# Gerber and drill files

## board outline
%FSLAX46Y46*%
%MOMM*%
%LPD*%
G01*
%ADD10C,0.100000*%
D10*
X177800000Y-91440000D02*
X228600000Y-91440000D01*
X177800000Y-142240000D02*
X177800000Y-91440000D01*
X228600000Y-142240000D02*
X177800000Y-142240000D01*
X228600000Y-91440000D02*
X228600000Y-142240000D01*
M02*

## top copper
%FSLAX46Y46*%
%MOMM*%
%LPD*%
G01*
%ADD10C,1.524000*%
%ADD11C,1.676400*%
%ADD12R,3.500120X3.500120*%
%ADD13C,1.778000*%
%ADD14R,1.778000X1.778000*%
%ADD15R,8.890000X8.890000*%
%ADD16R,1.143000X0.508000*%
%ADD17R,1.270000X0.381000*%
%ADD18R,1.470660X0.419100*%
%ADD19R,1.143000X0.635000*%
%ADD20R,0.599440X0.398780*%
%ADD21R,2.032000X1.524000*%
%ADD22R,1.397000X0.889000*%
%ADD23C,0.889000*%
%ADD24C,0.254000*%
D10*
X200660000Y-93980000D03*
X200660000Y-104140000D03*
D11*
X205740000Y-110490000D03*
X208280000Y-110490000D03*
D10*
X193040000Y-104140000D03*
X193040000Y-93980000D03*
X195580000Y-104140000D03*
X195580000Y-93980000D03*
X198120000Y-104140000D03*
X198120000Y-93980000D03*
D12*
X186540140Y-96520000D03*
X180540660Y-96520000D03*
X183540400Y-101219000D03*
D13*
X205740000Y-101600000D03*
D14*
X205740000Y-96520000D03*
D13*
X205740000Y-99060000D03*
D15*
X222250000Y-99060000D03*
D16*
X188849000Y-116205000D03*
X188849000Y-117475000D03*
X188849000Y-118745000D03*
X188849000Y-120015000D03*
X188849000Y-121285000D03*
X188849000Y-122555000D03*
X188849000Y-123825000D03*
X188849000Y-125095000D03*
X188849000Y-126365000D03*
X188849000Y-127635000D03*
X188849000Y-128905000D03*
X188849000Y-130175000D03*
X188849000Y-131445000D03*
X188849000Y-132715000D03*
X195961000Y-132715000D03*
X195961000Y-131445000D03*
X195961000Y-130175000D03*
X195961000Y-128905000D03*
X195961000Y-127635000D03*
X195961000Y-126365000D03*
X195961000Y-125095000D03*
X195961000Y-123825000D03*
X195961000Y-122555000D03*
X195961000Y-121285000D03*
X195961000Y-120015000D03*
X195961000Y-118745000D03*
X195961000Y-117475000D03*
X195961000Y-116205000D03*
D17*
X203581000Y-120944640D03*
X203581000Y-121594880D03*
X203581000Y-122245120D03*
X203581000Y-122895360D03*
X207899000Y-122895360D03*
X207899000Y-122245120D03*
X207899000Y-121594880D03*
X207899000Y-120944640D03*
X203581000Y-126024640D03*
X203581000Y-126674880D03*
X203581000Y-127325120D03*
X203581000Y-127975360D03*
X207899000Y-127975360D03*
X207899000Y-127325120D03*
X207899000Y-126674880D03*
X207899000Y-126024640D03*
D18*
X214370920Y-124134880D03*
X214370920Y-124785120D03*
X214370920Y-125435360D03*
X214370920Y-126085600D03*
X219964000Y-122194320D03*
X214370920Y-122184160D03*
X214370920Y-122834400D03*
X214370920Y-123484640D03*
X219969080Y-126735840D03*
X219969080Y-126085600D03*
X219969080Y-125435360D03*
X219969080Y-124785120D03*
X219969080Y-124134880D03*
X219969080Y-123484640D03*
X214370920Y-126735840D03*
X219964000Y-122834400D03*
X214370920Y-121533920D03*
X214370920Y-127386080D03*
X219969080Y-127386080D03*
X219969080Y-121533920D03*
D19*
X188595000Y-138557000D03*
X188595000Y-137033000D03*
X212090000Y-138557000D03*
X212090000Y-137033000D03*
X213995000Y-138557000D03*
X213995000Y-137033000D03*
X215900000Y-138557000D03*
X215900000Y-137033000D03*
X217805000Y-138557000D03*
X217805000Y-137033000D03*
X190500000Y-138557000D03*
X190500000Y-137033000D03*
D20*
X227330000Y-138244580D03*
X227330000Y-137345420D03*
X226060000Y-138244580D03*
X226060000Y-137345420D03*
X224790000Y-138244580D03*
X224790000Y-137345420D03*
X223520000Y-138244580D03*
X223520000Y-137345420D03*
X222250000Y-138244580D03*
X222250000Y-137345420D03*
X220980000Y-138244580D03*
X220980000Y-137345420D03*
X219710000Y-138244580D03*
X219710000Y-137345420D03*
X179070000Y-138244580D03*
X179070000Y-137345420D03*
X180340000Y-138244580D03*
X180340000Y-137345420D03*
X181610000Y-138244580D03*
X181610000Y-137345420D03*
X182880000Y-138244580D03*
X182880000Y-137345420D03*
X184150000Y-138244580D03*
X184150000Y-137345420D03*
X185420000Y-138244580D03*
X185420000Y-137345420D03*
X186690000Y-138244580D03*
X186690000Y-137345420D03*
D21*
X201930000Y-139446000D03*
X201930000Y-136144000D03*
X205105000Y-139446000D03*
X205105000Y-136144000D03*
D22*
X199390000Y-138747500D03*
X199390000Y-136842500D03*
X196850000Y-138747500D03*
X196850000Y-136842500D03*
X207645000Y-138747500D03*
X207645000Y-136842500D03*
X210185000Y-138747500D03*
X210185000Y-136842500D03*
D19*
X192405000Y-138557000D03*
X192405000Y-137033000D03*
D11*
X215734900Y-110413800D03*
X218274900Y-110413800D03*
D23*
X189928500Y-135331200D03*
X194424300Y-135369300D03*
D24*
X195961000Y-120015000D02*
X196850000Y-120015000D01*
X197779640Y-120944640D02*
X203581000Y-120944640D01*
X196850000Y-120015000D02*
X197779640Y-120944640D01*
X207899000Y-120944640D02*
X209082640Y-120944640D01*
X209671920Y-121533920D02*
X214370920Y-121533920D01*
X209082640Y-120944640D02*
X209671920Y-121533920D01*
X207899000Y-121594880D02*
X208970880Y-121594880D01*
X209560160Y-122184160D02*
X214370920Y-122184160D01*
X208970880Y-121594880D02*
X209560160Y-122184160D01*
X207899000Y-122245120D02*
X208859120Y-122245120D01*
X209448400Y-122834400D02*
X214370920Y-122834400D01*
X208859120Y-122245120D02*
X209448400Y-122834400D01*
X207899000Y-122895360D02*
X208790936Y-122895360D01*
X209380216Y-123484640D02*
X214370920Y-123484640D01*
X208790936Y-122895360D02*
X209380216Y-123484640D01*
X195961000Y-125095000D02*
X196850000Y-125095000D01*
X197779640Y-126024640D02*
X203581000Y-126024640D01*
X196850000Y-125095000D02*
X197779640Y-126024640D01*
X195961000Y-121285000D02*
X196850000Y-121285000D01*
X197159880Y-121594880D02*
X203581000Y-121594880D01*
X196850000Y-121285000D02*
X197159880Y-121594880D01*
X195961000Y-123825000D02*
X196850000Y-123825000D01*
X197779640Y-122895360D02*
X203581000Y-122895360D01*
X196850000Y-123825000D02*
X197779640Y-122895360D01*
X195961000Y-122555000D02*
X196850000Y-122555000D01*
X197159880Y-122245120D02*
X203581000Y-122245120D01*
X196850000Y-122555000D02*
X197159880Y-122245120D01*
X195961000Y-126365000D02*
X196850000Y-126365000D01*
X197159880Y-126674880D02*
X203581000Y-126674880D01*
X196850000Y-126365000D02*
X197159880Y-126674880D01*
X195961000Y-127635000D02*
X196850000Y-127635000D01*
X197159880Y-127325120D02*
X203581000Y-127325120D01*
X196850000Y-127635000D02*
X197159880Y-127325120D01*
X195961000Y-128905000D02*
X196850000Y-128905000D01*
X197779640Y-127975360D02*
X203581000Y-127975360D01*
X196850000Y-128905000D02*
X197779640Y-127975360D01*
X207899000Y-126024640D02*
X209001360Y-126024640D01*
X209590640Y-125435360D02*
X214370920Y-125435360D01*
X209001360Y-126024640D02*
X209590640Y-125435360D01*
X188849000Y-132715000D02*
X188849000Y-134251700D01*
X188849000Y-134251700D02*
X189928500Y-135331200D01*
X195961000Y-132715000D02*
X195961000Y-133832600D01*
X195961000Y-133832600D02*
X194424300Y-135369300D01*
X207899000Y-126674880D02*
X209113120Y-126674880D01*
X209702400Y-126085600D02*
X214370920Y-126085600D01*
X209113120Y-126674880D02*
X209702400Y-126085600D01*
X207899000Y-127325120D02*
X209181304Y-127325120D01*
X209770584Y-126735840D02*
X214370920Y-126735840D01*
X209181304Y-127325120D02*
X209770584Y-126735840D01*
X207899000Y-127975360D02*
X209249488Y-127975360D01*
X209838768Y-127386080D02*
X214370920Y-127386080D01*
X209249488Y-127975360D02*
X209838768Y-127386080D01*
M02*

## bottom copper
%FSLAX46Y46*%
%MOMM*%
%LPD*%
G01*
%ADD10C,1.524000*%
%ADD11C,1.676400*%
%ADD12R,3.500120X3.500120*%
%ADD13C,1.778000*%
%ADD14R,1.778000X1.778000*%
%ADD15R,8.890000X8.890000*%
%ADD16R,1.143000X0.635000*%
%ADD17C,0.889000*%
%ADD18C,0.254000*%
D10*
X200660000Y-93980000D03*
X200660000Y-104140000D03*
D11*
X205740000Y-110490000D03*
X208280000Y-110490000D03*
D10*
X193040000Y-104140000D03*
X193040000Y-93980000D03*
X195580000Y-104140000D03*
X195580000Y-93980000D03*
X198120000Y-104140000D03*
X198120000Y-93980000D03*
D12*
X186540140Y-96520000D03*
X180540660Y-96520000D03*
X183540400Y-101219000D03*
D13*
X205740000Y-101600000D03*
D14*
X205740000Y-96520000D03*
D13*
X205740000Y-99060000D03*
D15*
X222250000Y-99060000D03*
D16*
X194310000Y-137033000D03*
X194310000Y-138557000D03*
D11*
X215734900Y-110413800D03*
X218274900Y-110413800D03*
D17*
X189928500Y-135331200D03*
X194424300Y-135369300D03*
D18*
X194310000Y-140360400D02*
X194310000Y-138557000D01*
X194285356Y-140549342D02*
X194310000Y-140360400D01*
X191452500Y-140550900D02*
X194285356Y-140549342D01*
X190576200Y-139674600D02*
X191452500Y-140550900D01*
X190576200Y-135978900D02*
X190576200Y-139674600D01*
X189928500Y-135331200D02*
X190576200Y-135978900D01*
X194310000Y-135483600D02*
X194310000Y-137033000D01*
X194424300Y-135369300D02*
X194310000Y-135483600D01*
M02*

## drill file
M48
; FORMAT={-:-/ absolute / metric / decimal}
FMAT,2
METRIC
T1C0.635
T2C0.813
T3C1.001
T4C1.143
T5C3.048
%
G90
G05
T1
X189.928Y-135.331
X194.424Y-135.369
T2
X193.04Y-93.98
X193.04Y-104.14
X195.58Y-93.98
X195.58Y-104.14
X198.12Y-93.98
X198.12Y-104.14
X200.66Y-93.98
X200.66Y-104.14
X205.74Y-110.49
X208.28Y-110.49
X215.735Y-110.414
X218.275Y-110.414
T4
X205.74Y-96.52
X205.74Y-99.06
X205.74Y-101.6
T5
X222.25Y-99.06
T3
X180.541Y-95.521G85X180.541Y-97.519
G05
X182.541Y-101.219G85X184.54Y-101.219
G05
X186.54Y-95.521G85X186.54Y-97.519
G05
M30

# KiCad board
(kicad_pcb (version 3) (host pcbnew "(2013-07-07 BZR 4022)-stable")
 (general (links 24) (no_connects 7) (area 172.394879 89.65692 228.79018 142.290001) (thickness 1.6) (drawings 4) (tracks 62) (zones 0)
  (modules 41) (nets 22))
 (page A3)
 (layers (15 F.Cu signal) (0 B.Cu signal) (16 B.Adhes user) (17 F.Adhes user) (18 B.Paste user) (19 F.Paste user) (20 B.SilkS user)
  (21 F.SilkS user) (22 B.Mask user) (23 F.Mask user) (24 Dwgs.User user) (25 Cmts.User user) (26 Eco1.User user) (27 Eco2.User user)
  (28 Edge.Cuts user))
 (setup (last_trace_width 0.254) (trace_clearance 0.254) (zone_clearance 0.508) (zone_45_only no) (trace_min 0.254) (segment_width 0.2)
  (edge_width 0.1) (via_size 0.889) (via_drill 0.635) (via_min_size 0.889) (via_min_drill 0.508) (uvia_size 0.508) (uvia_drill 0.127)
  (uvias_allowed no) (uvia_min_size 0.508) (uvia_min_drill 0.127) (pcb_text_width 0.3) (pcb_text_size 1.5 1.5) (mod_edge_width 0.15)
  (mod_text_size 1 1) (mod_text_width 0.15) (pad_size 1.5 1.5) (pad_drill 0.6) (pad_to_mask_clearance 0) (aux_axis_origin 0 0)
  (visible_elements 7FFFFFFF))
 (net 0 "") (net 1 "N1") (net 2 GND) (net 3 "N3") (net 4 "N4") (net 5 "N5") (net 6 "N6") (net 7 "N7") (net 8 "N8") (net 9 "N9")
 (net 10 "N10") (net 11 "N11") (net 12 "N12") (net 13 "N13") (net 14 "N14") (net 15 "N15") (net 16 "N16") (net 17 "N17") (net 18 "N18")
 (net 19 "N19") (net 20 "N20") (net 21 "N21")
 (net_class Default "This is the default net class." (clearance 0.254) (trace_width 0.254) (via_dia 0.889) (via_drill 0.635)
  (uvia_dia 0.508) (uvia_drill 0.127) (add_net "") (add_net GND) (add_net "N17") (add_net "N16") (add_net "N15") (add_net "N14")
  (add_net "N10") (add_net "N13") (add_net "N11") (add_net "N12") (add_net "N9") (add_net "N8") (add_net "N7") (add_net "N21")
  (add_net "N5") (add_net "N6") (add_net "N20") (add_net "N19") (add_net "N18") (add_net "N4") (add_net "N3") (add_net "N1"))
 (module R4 (layer F.Cu) (at 200.66 99.06 270) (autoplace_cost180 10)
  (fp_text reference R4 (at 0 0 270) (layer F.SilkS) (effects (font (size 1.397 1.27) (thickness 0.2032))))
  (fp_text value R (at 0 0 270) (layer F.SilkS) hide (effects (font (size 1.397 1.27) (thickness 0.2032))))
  (pad 1 thru_hole circle (at -5.08 0 270) (size 1.524 1.524) (drill 0.8128) (layers *.Cu *.Mask F.SilkS) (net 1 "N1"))
  (pad 2 thru_hole circle (at 5.08 0 270) (size 1.524 1.524) (drill 0.8128) (layers *.Cu *.Mask F.SilkS) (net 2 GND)))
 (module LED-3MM (layer F.Cu) (at 207.01 110.49)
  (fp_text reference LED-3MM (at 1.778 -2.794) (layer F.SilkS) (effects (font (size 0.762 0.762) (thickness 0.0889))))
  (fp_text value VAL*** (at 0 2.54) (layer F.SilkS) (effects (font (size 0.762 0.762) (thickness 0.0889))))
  (pad 1 thru_hole circle (at -1.27 0) (size 1.6764 1.6764) (drill 0.8128) (layers *.Cu *.Mask F.SilkS))
  (pad 2 thru_hole circle (at 1.27 0) (size 1.6764 1.6764) (drill 0.8128) (layers *.Cu *.Mask F.SilkS)))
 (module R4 (layer F.Cu) (at 193.04 99.06 90) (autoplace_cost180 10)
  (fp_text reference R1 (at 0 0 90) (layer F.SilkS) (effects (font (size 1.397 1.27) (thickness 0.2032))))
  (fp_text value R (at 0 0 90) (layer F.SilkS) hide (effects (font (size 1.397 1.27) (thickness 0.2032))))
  (pad 1 thru_hole circle (at -5.08 0 90) (size 1.524 1.524) (drill 0.8128) (layers *.Cu *.Mask F.SilkS) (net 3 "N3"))
  (pad 2 thru_hole circle (at 5.08 0 90) (size 1.524 1.524) (drill 0.8128) (layers *.Cu *.Mask F.SilkS) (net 2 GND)))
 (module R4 (layer F.Cu) (at 195.58 99.06 90) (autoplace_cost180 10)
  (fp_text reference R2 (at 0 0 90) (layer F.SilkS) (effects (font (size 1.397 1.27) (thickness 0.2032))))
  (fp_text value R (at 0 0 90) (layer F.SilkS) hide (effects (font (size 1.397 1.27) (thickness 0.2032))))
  (pad 1 thru_hole circle (at -5.08 0 90) (size 1.524 1.524) (drill 0.8128) (layers *.Cu *.Mask F.SilkS) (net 2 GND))
  (pad 2 thru_hole circle (at 5.08 0 90) (size 1.524 1.524) (drill 0.8128) (layers *.Cu *.Mask F.SilkS) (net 2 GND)))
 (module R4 (layer F.Cu) (at 198.12 99.06 90) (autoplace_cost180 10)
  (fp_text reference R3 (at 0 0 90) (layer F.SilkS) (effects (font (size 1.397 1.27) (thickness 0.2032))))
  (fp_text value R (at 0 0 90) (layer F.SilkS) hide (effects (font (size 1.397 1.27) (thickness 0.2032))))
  (pad 1 thru_hole circle (at -5.08 0 90) (size 1.524 1.524) (drill 0.8128) (layers *.Cu *.Mask F.SilkS) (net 2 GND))
  (pad 2 thru_hole circle (at 5.08 0 90) (size 1.524 1.524) (drill 0.8128) (layers *.Cu *.Mask F.SilkS) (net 2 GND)))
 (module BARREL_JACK (layer F.Cu) (at 180.34 96.52)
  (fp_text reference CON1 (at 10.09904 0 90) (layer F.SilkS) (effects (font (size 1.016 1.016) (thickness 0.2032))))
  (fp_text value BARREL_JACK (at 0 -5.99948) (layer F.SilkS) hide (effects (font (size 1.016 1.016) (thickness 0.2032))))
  (pad 1 thru_hole rect (at 6.20014 0) (size 3.50012 3.50012) (drill oval 1.00076 2.99974) (layers *.Cu *.Mask F.SilkS) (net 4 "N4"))
  (pad 2 thru_hole rect (at 0.20066 0) (size 3.50012 3.50012) (drill oval 1.00076 2.99974) (layers *.Cu *.Mask F.SilkS) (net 2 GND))
  (pad 3 thru_hole rect (at 3.2004 4.699) (size 3.50012 3.50012) (drill oval 2.99974 1.00076) (layers *.Cu *.Mask F.SilkS) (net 2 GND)))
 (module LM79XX (layer F.Cu) (at 205.74 99.06)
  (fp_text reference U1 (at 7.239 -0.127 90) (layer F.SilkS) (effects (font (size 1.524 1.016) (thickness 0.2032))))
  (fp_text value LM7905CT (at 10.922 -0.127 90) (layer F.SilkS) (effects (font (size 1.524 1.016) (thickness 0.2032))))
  (pad VO thru_hole circle (at 0 2.54) (size 1.778 1.778) (drill 1.143) (layers *.Cu *.Mask F.SilkS))
  (pad GND thru_hole rect (at 0 -2.54) (size 1.778 1.778) (drill 1.143) (layers *.Cu *.Mask F.SilkS))
  (pad VI thru_hole circle (at 0 0) (size 1.778 1.778) (drill 1.143) (layers *.Cu *.Mask F.SilkS))
  (pad 4 thru_hole rect (at 16.51 0) (size 8.89 8.89) (drill 3.048) (layers *.Cu *.SilkS *.Mask)))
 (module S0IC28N (layer F.Cu) (at 192.405 124.46 270)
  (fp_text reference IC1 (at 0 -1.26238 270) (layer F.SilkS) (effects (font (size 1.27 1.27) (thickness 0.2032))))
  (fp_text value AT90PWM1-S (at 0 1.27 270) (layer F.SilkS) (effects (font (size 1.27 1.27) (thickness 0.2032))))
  (pad 1 smd rect (at -8.255 3.556 270) (size 0.508 1.143) (layers F.Cu F.Paste F.Mask))
  (pad 2 smd rect (at -6.985 3.556 270) (size 0.508 1.143) (layers F.Cu F.Paste F.Mask))
  (pad 3 smd rect (at -5.715 3.556 270) (size 0.508 1.143) (layers F.Cu F.Paste F.Mask))
  (pad 4 smd rect (at -4.445 3.556 270) (size 0.508 1.143) (layers F.Cu F.Paste F.Mask))
  (pad 5 smd rect (at -3.175 3.556 270) (size 0.508 1.143) (layers F.Cu F.Paste F.Mask))
  (pad 6 smd rect (at -1.905 3.556 270) (size 0.508 1.143) (layers F.Cu F.Paste F.Mask))
  (pad 7 smd rect (at -0.635 3.556 270) (size 0.508 1.143) (layers F.Cu F.Paste F.Mask))
  (pad 8 smd rect (at 0.635 3.556 270) (size 0.508 1.143) (layers F.Cu F.Paste F.Mask))
  (pad 9 smd rect (at 1.905 3.556 270) (size 0.508 1.143) (layers F.Cu F.Paste F.Mask))
  (pad 10 smd rect (at 3.175 3.556 270) (size 0.508 1.143) (layers F.Cu F.Paste F.Mask))
  (pad 11 smd rect (at 4.445 3.556 270) (size 0.508 1.143) (layers F.Cu F.Paste F.Mask))
  (pad 12 smd rect (at 5.715 3.556 270) (size 0.508 1.143) (layers F.Cu F.Paste F.Mask))
  (pad 13 smd rect (at 6.985 3.556 270) (size 0.508 1.143) (layers F.Cu F.Paste F.Mask))
  (pad 14 smd rect (at 8.255 3.556 270) (size 0.508 1.143) (layers F.Cu F.Paste F.Mask) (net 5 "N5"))
  (pad 15 smd rect (at 8.255 -3.556 270) (size 0.508 1.143) (layers F.Cu F.Paste F.Mask) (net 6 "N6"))
  (pad 16 smd rect (at 6.985 -3.556 270) (size 0.508 1.143) (layers F.Cu F.Paste F.Mask))
  (pad 17 smd rect (at 5.715 -3.556 270) (size 0.508 1.143) (layers F.Cu F.Paste F.Mask))
  (pad 18 smd rect (at 4.445 -3.556 270) (size 0.508 1.143) (layers F.Cu F.Paste F.Mask) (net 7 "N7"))
  (pad 19 smd rect (at 3.175 -3.556 270) (size 0.508 1.143) (layers F.Cu F.Paste F.Mask) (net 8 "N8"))
  (pad 20 smd rect (at 1.905 -3.556 270) (size 0.508 1.143) (layers F.Cu F.Paste F.Mask) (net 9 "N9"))
  (pad 21 smd rect (at 0.635 -3.556 270) (size 0.508 1.143) (layers F.Cu F.Paste F.Mask) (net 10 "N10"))
  (pad 22 smd rect (at -0.635 -3.556 270) (size 0.508 1.143) (layers F.Cu F.Paste F.Mask) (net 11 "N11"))
  (pad 23 smd rect (at -1.905 -3.556 270) (size 0.508 1.143) (layers F.Cu F.Paste F.Mask) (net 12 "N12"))
  (pad 24 smd rect (at -3.175 -3.556 270) (size 0.508 1.143) (layers F.Cu F.Paste F.Mask) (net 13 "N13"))
  (pad 25 smd rect (at -4.445 -3.556 270) (size 0.508 1.143) (layers F.Cu F.Paste F.Mask))
  (pad 26 smd rect (at -5.715 -3.556 270) (size 0.508 1.143) (layers F.Cu F.Paste F.Mask))
  (pad 27 smd rect (at -6.985 -3.556 270) (size 0.508 1.143) (layers F.Cu F.Paste F.Mask))
  (pad 28 smd rect (at -8.255 -3.556 270) (size 0.508 1.143) (layers F.Cu F.Paste F.Mask)))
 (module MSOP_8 (layer F.Cu) (at 205.74 121.92 270)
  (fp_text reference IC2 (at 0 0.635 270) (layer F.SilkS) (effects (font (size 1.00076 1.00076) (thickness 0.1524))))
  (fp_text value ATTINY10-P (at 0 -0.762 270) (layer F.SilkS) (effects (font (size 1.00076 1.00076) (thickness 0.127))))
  (pad 1 smd rect (at -0.97536 2.159 270) (size 0.381 1.27) (layers F.Cu F.Paste F.Mask))
  (pad 2 smd rect (at -0.32512 2.159 270) (size 0.381 1.27) (layers F.Cu F.Paste F.Mask) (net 13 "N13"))
  (pad 3 smd rect (at 0.32512 2.159 270) (size 0.381 1.27) (layers F.Cu F.Paste F.Mask) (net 12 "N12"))
  (pad 4 smd rect (at 0.97536 2.159 270) (size 0.381 1.27) (layers F.Cu F.Paste F.Mask) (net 11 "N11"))
  (pad 5 smd rect (at 0.97536 -2.159 270) (size 0.381 1.27) (layers F.Cu F.Paste F.Mask) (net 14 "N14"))
  (pad 6 smd rect (at 0.32512 -2.159 270) (size 0.381 1.27) (layers F.Cu F.Paste F.Mask) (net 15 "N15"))
  (pad 7 smd rect (at -0.32512 -2.159 270) (size 0.381 1.27) (layers F.Cu F.Paste F.Mask) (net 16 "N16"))
  (pad 8 smd rect (at -0.97536 -2.159 270) (size 0.381 1.27) (layers F.Cu F.Paste F.Mask) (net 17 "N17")))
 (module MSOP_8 (layer F.Cu) (at 205.74 127 270)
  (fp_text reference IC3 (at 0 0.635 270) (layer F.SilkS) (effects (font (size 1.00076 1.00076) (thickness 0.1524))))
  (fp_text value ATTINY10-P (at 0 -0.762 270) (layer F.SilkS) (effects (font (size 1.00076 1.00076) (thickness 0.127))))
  (pad 1 smd rect (at -0.97536 2.159 270) (size 0.381 1.27) (layers F.Cu F.Paste F.Mask) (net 10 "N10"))
  (pad 2 smd rect (at -0.32512 2.159 270) (size 0.381 1.27) (layers F.Cu F.Paste F.Mask) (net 9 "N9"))
  (pad 3 smd rect (at 0.32512 2.159 270) (size 0.381 1.27) (layers F.Cu F.Paste F.Mask) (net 8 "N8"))
  (pad 4 smd rect (at 0.97536 2.159 270) (size 0.381 1.27) (layers F.Cu F.Paste F.Mask) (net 7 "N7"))
  (pad 5 smd rect (at 0.97536 -2.159 270) (size 0.381 1.27) (layers F.Cu F.Paste F.Mask) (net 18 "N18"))
  (pad 6 smd rect (at 0.32512 -2.159 270) (size 0.381 1.27) (layers F.Cu F.Paste F.Mask) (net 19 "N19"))
  (pad 7 smd rect (at -0.32512 -2.159 270) (size 0.381 1.27) (layers F.Cu F.Paste F.Mask) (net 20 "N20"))
  (pad 8 smd rect (at -0.97536 -2.159 270) (size 0.381 1.27) (layers F.Cu F.Paste F.Mask) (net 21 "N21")))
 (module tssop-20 (layer F.Cu) (at 217.17 124.46 270)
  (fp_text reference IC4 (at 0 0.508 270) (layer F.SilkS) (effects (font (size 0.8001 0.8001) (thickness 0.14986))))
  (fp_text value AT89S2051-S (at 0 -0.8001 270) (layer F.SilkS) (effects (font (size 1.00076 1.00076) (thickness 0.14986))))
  (pad 5 smd rect (at -0.32512 2.79908 270) (size 0.4191 1.47066) (layers F.Cu F.Paste F.Mask))
  (pad 6 smd rect (at 0.32512 2.79908 270) (size 0.4191 1.47066) (layers F.Cu F.Paste F.Mask))
  (pad 7 smd rect (at 0.97536 2.79908 270) (size 0.4191 1.47066) (layers F.Cu F.Paste F.Mask) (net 21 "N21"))
  (pad 8 smd rect (at 1.6256 2.79908 270) (size 0.4191 1.47066) (layers F.Cu F.Paste F.Mask) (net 20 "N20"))
  (pad 19 smd rect (at -2.26568 -2.794 270) (size 0.4191 1.47066) (layers F.Cu F.Paste F.Mask))
  (pad 2 smd rect (at -2.27584 2.79908 270) (size 0.4191 1.47066) (layers F.Cu F.Paste F.Mask) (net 16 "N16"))
  (pad 3 smd rect (at -1.6256 2.79908 270) (size 0.4191 1.47066) (layers F.Cu F.Paste F.Mask) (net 15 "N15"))
  (pad 4 smd rect (at -0.97536 2.79908 270) (size 0.4191 1.47066) (layers F.Cu F.Paste F.Mask) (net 14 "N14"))
  (pad 12 smd rect (at 2.27584 -2.79908 270) (size 0.4191 1.47066) (layers F.Cu F.Paste F.Mask))
  (pad 13 smd rect (at 1.6256 -2.79908 270) (size 0.4191 1.47066) (layers F.Cu F.Paste F.Mask))
  (pad 14 smd rect (at 0.97536 -2.79908 270) (size 0.4191 1.47066) (layers F.Cu F.Paste F.Mask))
  (pad 15 smd rect (at 0.32512 -2.79908 270) (size 0.4191 1.47066) (layers F.Cu F.Paste F.Mask))
  (pad 16 smd rect (at -0.32512 -2.79908 270) (size 0.4191 1.47066) (layers F.Cu F.Paste F.Mask))
  (pad 17 smd rect (at -0.97536 -2.79908 270) (size 0.4191 1.47066) (layers F.Cu F.Paste F.Mask))
  (pad 9 smd rect (at 2.27584 2.79908 270) (size 0.4191 1.47066) (layers F.Cu F.Paste F.Mask) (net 19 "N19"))
  (pad 18 smd rect (at -1.6256 -2.794 270) (size 0.4191 1.47066) (layers F.Cu F.Paste F.Mask))
  (pad 1 smd rect (at -2.92608 2.79908 270) (size 0.4191 1.47066) (layers F.Cu F.Paste F.Mask) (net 17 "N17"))
  (pad 10 smd rect (at 2.92608 2.79908 270) (size 0.4191 1.47066) (layers F.Cu F.Paste F.Mask) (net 18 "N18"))
  (pad 11 smd rect (at 2.92608 -2.79908 270) (size 0.4191 1.47066) (layers F.Cu F.Paste F.Mask))
  (pad 20 smd rect (at -2.92608 -2.79908 270) (size 0.4191 1.47066) (layers F.Cu F.Paste F.Mask)))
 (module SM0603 (layer F.Cu) (at 188.595 137.795 90)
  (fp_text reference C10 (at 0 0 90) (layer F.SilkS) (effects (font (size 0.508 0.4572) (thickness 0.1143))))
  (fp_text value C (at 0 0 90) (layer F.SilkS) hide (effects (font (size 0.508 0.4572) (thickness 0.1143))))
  (pad 1 smd rect (at -0.762 0 90) (size 0.635 1.143) (layers F.Cu F.Paste F.Mask))
  (pad 2 smd rect (at 0.762 0 90) (size 0.635 1.143) (layers F.Cu F.Paste F.Mask)))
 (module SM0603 (layer F.Cu) (at 212.09 137.795 90)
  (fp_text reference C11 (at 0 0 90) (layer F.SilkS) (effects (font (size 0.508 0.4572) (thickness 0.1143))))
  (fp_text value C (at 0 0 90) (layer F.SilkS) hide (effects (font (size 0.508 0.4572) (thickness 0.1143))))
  (pad 1 smd rect (at -0.762 0 90) (size 0.635 1.143) (layers F.Cu F.Paste F.Mask))
  (pad 2 smd rect (at 0.762 0 90) (size 0.635 1.143) (layers F.Cu F.Paste F.Mask)))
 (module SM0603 (layer F.Cu) (at 213.995 137.795 90)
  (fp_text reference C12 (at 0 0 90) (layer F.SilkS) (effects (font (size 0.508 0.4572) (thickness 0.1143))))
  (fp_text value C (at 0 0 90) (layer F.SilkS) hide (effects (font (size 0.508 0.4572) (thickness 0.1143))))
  (pad 1 smd rect (at -0.762 0 90) (size 0.635 1.143) (layers F.Cu F.Paste F.Mask))
  (pad 2 smd rect (at 0.762 0 90) (size 0.635 1.143) (layers F.Cu F.Paste F.Mask)))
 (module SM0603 (layer F.Cu) (at 215.9 137.795 90)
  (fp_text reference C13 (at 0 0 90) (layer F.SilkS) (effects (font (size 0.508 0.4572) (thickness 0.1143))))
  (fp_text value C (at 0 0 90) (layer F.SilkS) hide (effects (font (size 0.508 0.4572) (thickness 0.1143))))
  (pad 1 smd rect (at -0.762 0 90) (size 0.635 1.143) (layers F.Cu F.Paste F.Mask))
  (pad 2 smd rect (at 0.762 0 90) (size 0.635 1.143) (layers F.Cu F.Paste F.Mask)))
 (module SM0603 (layer F.Cu) (at 217.805 137.795 90)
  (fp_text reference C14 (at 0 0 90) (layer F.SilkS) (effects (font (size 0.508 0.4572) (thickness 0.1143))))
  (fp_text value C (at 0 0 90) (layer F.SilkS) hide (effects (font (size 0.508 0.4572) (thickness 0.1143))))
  (pad 1 smd rect (at -0.762 0 90) (size 0.635 1.143) (layers F.Cu F.Paste F.Mask))
  (pad 2 smd rect (at 0.762 0 90) (size 0.635 1.143) (layers F.Cu F.Paste F.Mask)))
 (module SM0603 (layer F.Cu) (at 190.5 137.795 90)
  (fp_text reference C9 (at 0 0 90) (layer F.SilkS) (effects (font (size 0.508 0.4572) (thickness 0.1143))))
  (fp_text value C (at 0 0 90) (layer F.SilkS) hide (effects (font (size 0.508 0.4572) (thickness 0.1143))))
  (pad 1 smd rect (at -0.762 0 90) (size 0.635 1.143) (layers F.Cu F.Paste F.Mask))
  (pad 2 smd rect (at 0.762 0 90) (size 0.635 1.143) (layers F.Cu F.Paste F.Mask)))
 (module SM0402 (layer F.Cu) (at 227.33 137.795 90)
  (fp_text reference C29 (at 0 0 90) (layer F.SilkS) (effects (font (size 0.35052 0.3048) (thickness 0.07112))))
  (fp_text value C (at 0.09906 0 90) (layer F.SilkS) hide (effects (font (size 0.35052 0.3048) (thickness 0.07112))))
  (pad 1 smd rect (at -0.44958 0 90) (size 0.39878 0.59944) (layers F.Cu F.Paste F.Mask))
  (pad 2 smd rect (at 0.44958 0 90) (size 0.39878 0.59944) (layers F.Cu F.Paste F.Mask)))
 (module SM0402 (layer F.Cu) (at 226.06 137.795 90)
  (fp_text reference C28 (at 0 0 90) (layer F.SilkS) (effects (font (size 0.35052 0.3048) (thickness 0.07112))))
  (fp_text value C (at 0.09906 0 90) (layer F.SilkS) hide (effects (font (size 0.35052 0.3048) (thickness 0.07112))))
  (pad 1 smd rect (at -0.44958 0 90) (size 0.39878 0.59944) (layers F.Cu F.Paste F.Mask))
  (pad 2 smd rect (at 0.44958 0 90) (size 0.39878 0.59944) (layers F.Cu F.Paste F.Mask)))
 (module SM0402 (layer F.Cu) (at 224.79 137.795 90)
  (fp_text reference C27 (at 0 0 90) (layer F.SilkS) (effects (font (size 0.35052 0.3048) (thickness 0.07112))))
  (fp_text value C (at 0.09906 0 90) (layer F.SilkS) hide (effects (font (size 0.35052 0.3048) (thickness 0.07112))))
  (pad 1 smd rect (at -0.44958 0 90) (size 0.39878 0.59944) (layers F.Cu F.Paste F.Mask))
  (pad 2 smd rect (at 0.44958 0 90) (size 0.39878 0.59944) (layers F.Cu F.Paste F.Mask)))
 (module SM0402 (layer F.Cu) (at 223.52 137.795 90)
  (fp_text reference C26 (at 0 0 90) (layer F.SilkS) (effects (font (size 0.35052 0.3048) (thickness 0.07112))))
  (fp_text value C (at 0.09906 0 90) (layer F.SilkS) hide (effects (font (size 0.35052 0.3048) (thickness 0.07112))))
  (pad 1 smd rect (at -0.44958 0 90) (size 0.39878 0.59944) (layers F.Cu F.Paste F.Mask))
  (pad 2 smd rect (at 0.44958 0 90) (size 0.39878 0.59944) (layers F.Cu F.Paste F.Mask)))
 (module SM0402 (layer F.Cu) (at 222.25 137.795 90)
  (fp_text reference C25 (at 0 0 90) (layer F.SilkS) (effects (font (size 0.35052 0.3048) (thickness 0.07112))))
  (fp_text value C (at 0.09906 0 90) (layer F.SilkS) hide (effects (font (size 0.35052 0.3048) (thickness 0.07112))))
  (pad 1 smd rect (at -0.44958 0 90) (size 0.39878 0.59944) (layers F.Cu F.Paste F.Mask))
  (pad 2 smd rect (at 0.44958 0 90) (size 0.39878 0.59944) (layers F.Cu F.Paste F.Mask)))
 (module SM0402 (layer F.Cu) (at 220.98 137.795 90)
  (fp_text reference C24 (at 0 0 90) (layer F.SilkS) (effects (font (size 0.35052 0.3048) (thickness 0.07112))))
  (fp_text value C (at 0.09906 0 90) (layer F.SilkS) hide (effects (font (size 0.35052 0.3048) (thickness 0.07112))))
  (pad 1 smd rect (at -0.44958 0 90) (size 0.39878 0.59944) (layers F.Cu F.Paste F.Mask))
  (pad 2 smd rect (at 0.44958 0 90) (size 0.39878 0.59944) (layers F.Cu F.Paste F.Mask)))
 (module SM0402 (layer F.Cu) (at 219.71 137.795 90)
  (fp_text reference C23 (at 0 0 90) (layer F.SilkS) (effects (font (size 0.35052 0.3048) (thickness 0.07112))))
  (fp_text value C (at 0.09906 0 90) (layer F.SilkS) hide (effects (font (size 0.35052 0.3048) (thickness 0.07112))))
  (pad 1 smd rect (at -0.44958 0 90) (size 0.39878 0.59944) (layers F.Cu F.Paste F.Mask))
  (pad 2 smd rect (at 0.44958 0 90) (size 0.39878 0.59944) (layers F.Cu F.Paste F.Mask)))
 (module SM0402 (layer F.Cu) (at 179.07 137.795 90)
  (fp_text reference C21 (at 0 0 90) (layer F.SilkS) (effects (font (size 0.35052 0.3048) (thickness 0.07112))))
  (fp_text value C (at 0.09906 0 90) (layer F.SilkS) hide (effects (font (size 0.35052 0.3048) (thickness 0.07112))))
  (pad 1 smd rect (at -0.44958 0 90) (size 0.39878 0.59944) (layers F.Cu F.Paste F.Mask))
  (pad 2 smd rect (at 0.44958 0 90) (size 0.39878 0.59944) (layers F.Cu F.Paste F.Mask)))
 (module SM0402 (layer F.Cu) (at 180.34 137.795 90)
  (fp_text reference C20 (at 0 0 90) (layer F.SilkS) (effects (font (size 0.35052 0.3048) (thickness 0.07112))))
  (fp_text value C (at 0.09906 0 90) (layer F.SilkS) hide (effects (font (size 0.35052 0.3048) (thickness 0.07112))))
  (pad 1 smd rect (at -0.44958 0 90) (size 0.39878 0.59944) (layers F.Cu F.Paste F.Mask))
  (pad 2 smd rect (at 0.44958 0 90) (size 0.39878 0.59944) (layers F.Cu F.Paste F.Mask)))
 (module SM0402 (layer F.Cu) (at 181.61 137.795 90)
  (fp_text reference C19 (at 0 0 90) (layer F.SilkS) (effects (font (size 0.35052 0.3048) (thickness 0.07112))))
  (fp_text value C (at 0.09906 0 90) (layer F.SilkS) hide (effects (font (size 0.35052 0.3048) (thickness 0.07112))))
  (pad 1 smd rect (at -0.44958 0 90) (size 0.39878 0.59944) (layers F.Cu F.Paste F.Mask))
  (pad 2 smd rect (at 0.44958 0 90) (size 0.39878 0.59944) (layers F.Cu F.Paste F.Mask)))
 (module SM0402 (layer F.Cu) (at 182.88 137.795 90)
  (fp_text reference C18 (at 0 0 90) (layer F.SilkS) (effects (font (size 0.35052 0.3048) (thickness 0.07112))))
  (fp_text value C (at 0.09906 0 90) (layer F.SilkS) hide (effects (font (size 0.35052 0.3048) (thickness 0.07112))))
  (pad 1 smd rect (at -0.44958 0 90) (size 0.39878 0.59944) (layers F.Cu F.Paste F.Mask))
  (pad 2 smd rect (at 0.44958 0 90) (size 0.39878 0.59944) (layers F.Cu F.Paste F.Mask)))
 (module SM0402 (layer F.Cu) (at 184.15 137.795 90)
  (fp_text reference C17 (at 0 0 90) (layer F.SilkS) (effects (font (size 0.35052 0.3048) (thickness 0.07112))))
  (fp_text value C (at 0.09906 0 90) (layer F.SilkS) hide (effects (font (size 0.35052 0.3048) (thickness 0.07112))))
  (pad 1 smd rect (at -0.44958 0 90) (size 0.39878 0.59944) (layers F.Cu F.Paste F.Mask))
  (pad 2 smd rect (at 0.44958 0 90) (size 0.39878 0.59944) (layers F.Cu F.Paste F.Mask)))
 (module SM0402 (layer F.Cu) (at 185.42 137.795 90)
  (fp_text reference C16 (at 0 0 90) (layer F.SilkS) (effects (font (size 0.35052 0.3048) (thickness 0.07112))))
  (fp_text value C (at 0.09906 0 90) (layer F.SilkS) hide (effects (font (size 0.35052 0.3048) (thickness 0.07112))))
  (pad 1 smd rect (at -0.44958 0 90) (size 0.39878 0.59944) (layers F.Cu F.Paste F.Mask))
  (pad 2 smd rect (at 0.44958 0 90) (size 0.39878 0.59944) (layers F.Cu F.Paste F.Mask)))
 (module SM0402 (layer F.Cu) (at 186.69 137.795 90)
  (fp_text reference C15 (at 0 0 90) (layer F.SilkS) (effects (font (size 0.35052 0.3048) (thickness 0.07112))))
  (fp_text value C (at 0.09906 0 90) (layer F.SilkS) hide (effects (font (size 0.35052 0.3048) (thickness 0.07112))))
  (pad 1 smd rect (at -0.44958 0 90) (size 0.39878 0.59944) (layers F.Cu F.Paste F.Mask))
  (pad 2 smd rect (at 0.44958 0 90) (size 0.39878 0.59944) (layers F.Cu F.Paste F.Mask)))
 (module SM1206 (layer F.Cu) (at 201.93 137.795 90)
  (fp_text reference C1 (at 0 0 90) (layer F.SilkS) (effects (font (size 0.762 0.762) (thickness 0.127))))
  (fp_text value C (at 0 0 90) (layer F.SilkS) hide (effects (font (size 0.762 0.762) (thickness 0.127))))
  (pad 1 smd rect (at -1.651 0 90) (size 1.524 2.032) (layers F.Cu F.Paste F.Mask))
  (pad 2 smd rect (at 1.651 0 90) (size 1.524 2.032) (layers F.Cu F.Paste F.Mask)))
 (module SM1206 (layer F.Cu) (at 205.105 137.795 90)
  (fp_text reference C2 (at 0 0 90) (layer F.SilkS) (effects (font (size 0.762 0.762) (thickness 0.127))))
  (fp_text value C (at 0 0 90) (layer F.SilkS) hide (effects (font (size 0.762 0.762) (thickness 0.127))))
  (pad 1 smd rect (at -1.651 0 90) (size 1.524 2.032) (layers F.Cu F.Paste F.Mask))
  (pad 2 smd rect (at 1.651 0 90) (size 1.524 2.032) (layers F.Cu F.Paste F.Mask)))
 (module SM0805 (layer F.Cu) (at 199.39 137.795 90)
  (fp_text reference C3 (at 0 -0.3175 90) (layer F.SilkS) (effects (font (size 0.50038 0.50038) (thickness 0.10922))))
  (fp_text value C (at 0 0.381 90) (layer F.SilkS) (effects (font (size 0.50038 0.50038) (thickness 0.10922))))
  (pad 1 smd rect (at -0.9525 0 90) (size 0.889 1.397) (layers F.Cu F.Paste F.Mask))
  (pad 2 smd rect (at 0.9525 0 90) (size 0.889 1.397) (layers F.Cu F.Paste F.Mask)))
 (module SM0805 (layer F.Cu) (at 196.85 137.795 90)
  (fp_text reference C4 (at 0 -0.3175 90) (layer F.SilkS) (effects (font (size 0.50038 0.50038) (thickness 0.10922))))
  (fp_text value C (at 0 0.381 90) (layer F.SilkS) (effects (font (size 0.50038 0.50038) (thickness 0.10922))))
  (pad 1 smd rect (at -0.9525 0 90) (size 0.889 1.397) (layers F.Cu F.Paste F.Mask))
  (pad 2 smd rect (at 0.9525 0 90) (size 0.889 1.397) (layers F.Cu F.Paste F.Mask)))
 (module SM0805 (layer F.Cu) (at 207.645 137.795 90)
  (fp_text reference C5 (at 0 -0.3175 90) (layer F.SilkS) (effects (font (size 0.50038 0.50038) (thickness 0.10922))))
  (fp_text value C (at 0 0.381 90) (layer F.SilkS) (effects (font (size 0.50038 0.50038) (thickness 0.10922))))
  (pad 1 smd rect (at -0.9525 0 90) (size 0.889 1.397) (layers F.Cu F.Paste F.Mask))
  (pad 2 smd rect (at 0.9525 0 90) (size 0.889 1.397) (layers F.Cu F.Paste F.Mask)))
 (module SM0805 (layer F.Cu) (at 210.185 137.795 90)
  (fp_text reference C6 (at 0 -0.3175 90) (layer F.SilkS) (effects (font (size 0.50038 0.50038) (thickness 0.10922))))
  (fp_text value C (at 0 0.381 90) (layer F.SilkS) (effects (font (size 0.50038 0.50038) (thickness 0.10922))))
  (pad 1 smd rect (at -0.9525 0 90) (size 0.889 1.397) (layers F.Cu F.Paste F.Mask))
  (pad 2 smd rect (at 0.9525 0 90) (size 0.889 1.397) (layers F.Cu F.Paste F.Mask)))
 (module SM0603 (layer B.Cu) (at 194.31 137.795 270)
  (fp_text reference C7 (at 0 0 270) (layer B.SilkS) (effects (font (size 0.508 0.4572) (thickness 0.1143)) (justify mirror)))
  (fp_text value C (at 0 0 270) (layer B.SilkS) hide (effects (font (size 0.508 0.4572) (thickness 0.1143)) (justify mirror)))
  (pad 1 smd rect (at -0.762 0 270) (size 0.635 1.143) (layers B.Cu B.Paste B.Mask) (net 6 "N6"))
  (pad 2 smd rect (at 0.762 0 270) (size 0.635 1.143) (layers B.Cu B.Paste B.Mask) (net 5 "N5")))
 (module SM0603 (layer F.Cu) (at 192.405 137.795 90)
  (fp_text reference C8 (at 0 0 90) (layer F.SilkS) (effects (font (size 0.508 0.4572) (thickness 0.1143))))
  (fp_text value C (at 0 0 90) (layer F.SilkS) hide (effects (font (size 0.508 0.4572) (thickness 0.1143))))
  (pad 1 smd rect (at -0.762 0 90) (size 0.635 1.143) (layers F.Cu F.Paste F.Mask))
  (pad 2 smd rect (at 0.762 0 90) (size 0.635 1.143) (layers F.Cu F.Paste F.Mask)))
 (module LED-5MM (layer F.Cu) (at 217.0049 110.4138)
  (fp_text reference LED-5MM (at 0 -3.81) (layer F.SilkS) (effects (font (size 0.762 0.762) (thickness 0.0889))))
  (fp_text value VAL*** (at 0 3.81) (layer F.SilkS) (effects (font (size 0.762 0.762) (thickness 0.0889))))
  (pad 1 thru_hole circle (at -1.27 0) (size 1.6764 1.6764) (drill 0.8128) (layers *.Cu *.Mask F.SilkS))
  (pad 2 thru_hole circle (at 1.27 0) (size 1.6764 1.6764) (drill 0.8128) (layers *.Cu *.Mask F.SilkS)))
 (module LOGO (layer F.Cu) (at 183.3118 109.6137)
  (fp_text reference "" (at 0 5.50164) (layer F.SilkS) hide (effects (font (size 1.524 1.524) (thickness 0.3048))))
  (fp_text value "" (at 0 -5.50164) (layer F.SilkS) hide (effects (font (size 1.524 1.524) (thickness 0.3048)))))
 (gr_line (start 177.8 91.44) (end 228.6 91.44) (angle 90) (layer Edge.Cuts) (width 0.1))
 (gr_line (start 177.8 142.24) (end 177.8 91.44) (angle 90) (layer Edge.Cuts) (width 0.1))
 (gr_line (start 228.6 142.24) (end 177.8 142.24) (angle 90) (layer Edge.Cuts) (width 0.1))
 (gr_line (start 228.6 91.44) (end 228.6 142.24) (angle 90) (layer Edge.Cuts) (width 0.1))
 (segment (start 195.961 120.015) (end 196.85 120.015) (width 0.254) (layer F.Cu) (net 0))
 (segment (start 197.77964 120.94464) (end 203.581 120.94464) (width 0.254) (layer F.Cu) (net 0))
 (segment (start 196.85 120.015) (end 197.77964 120.94464) (width 0.254) (layer F.Cu) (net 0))
 (segment (start 207.899 120.94464) (end 209.08264 120.94464) (width 0.254) (layer F.Cu) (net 17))
 (segment (start 209.67192 121.53392) (end 214.37092 121.53392) (width 0.254) (layer F.Cu) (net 17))
 (segment (start 209.08264 120.94464) (end 209.67192 121.53392) (width 0.254) (layer F.Cu) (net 17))
 (segment (start 207.899 121.59488) (end 208.97088 121.59488) (width 0.254) (layer F.Cu) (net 16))
 (segment (start 209.56016 122.18416) (end 214.37092 122.18416) (width 0.254) (layer F.Cu) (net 16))
 (segment (start 208.97088 121.59488) (end 209.56016 122.18416) (width 0.254) (layer F.Cu) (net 16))
 (segment (start 207.899 122.24512) (end 208.85912 122.24512) (width 0.254) (layer F.Cu) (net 15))
 (segment (start 209.4484 122.8344) (end 214.37092 122.8344) (width 0.254) (layer F.Cu) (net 15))
 (segment (start 208.85912 122.24512) (end 209.4484 122.8344) (width 0.254) (layer F.Cu) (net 15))
 (segment (start 207.899 122.89536) (end 208.790936 122.89536) (width 0.254) (layer F.Cu) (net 14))
 (segment (start 209.380216 123.48464) (end 214.37092 123.48464) (width 0.254) (layer F.Cu) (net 14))
 (segment (start 208.790936 122.89536) (end 209.380216 123.48464) (width 0.254) (layer F.Cu) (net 14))
 (segment (start 195.961 125.095) (end 196.85 125.095) (width 0.254) (layer F.Cu) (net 10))
 (segment (start 197.77964 126.02464) (end 203.581 126.02464) (width 0.254) (layer F.Cu) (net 10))
 (segment (start 196.85 125.095) (end 197.77964 126.02464) (width 0.254) (layer F.Cu) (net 10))
 (segment (start 195.961 121.285) (end 196.85 121.285) (width 0.254) (layer F.Cu) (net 13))
 (segment (start 197.15988 121.59488) (end 203.581 121.59488) (width 0.254) (layer F.Cu) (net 13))
 (segment (start 196.85 121.285) (end 197.15988 121.59488) (width 0.254) (layer F.Cu) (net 13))
 (segment (start 195.961 123.825) (end 196.85 123.825) (width 0.254) (layer F.Cu) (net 11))
 (segment (start 197.77964 122.89536) (end 203.581 122.89536) (width 0.254) (layer F.Cu) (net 11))
 (segment (start 196.85 123.825) (end 197.77964 122.89536) (width 0.254) (layer F.Cu) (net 11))
 (segment (start 195.961 122.555) (end 196.85 122.555) (width 0.254) (layer F.Cu) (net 12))
 (segment (start 197.15988 122.24512) (end 203.581 122.24512) (width 0.254) (layer F.Cu) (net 12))
 (segment (start 196.85 122.555) (end 197.15988 122.24512) (width 0.254) (layer F.Cu) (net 12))
 (segment (start 195.961 126.365) (end 196.85 126.365) (width 0.254) (layer F.Cu) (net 9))
 (segment (start 197.15988 126.67488) (end 203.581 126.67488) (width 0.254) (layer F.Cu) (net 9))
 (segment (start 196.85 126.365) (end 197.15988 126.67488) (width 0.254) (layer F.Cu) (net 9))
 (segment (start 195.961 127.635) (end 196.85 127.635) (width 0.254) (layer F.Cu) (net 8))
 (segment (start 197.15988 127.32512) (end 203.581 127.32512) (width 0.254) (layer F.Cu) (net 8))
 (segment (start 196.85 127.635) (end 197.15988 127.32512) (width 0.254) (layer F.Cu) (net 8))
 (segment (start 195.961 128.905) (end 196.85 128.905) (width 0.254) (layer F.Cu) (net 7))
 (segment (start 197.77964 127.97536) (end 203.581 127.97536) (width 0.254) (layer F.Cu) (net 7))
 (segment (start 196.85 128.905) (end 197.77964 127.97536) (width 0.254) (layer F.Cu) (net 7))
 (segment (start 207.899 126.02464) (end 209.00136 126.02464) (width 0.254) (layer F.Cu) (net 21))
 (segment (start 209.59064 125.43536) (end 214.37092 125.43536) (width 0.254) (layer F.Cu) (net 21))
 (segment (start 209.00136 126.02464) (end 209.59064 125.43536) (width 0.254) (layer F.Cu) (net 21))
 (segment (start 188.849 132.715) (end 188.849 134.2517) (width 0.254) (layer F.Cu) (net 5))
 (segment (start 194.31 140.3604) (end 194.31 138.557) (width 0.254) (layer B.Cu) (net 5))
 (segment (start 194.285356 140.549342) (end 194.31 140.3604) (width 0.254) (layer B.Cu) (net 5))
 (segment (start 191.4525 140.5509) (end 194.285356 140.549342) (width 0.254) (layer B.Cu) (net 5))
 (segment (start 190.5762 139.6746) (end 191.4525 140.5509) (width 0.254) (layer B.Cu) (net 5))
 (segment (start 190.5762 135.9789) (end 190.5762 139.6746) (width 0.254) (layer B.Cu) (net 5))
 (segment (start 189.9285 135.3312) (end 190.5762 135.9789) (width 0.254) (layer B.Cu) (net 5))
 (via (at 189.9285 135.3312) (size 0.889) (layers F.Cu B.Cu) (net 5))
 (segment (start 188.849 134.2517) (end 189.9285 135.3312) (width 0.254) (layer F.Cu) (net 5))
 (segment (start 195.961 132.715) (end 195.961 133.8326) (width 0.254) (layer F.Cu) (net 6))
 (segment (start 194.31 135.4836) (end 194.31 137.033) (width 0.254) (layer B.Cu) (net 6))
 (segment (start 194.4243 135.3693) (end 194.31 135.4836) (width 0.254) (layer B.Cu) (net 6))
 (via (at 194.4243 135.3693) (size 0.889) (layers F.Cu B.Cu) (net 6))
 (segment (start 195.961 133.8326) (end 194.4243 135.3693) (width 0.254) (layer F.Cu) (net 6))
 (segment (start 207.899 126.67488) (end 209.11312 126.67488) (width 0.254) (layer F.Cu) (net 20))
 (segment (start 209.7024 126.0856) (end 214.37092 126.0856) (width 0.254) (layer F.Cu) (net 20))
 (segment (start 209.11312 126.67488) (end 209.7024 126.0856) (width 0.254) (layer F.Cu) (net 20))
 (segment (start 207.899 127.32512) (end 209.181304 127.32512) (width 0.254) (layer F.Cu) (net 19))
 (segment (start 209.770584 126.73584) (end 214.37092 126.73584) (width 0.254) (layer F.Cu) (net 19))
 (segment (start 209.181304 127.32512) (end 209.770584 126.73584) (width 0.254) (layer F.Cu) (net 19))
 (segment (start 207.899 127.97536) (end 209.249488 127.97536) (width 0.254) (layer F.Cu) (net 18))
 (segment (start 209.838768 127.38608) (end 214.37092 127.38608) (width 0.254) (layer F.Cu) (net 18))
 (segment (start 209.249488 127.97536) (end 209.838768 127.38608) (width 0.254) (layer F.Cu) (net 18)))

